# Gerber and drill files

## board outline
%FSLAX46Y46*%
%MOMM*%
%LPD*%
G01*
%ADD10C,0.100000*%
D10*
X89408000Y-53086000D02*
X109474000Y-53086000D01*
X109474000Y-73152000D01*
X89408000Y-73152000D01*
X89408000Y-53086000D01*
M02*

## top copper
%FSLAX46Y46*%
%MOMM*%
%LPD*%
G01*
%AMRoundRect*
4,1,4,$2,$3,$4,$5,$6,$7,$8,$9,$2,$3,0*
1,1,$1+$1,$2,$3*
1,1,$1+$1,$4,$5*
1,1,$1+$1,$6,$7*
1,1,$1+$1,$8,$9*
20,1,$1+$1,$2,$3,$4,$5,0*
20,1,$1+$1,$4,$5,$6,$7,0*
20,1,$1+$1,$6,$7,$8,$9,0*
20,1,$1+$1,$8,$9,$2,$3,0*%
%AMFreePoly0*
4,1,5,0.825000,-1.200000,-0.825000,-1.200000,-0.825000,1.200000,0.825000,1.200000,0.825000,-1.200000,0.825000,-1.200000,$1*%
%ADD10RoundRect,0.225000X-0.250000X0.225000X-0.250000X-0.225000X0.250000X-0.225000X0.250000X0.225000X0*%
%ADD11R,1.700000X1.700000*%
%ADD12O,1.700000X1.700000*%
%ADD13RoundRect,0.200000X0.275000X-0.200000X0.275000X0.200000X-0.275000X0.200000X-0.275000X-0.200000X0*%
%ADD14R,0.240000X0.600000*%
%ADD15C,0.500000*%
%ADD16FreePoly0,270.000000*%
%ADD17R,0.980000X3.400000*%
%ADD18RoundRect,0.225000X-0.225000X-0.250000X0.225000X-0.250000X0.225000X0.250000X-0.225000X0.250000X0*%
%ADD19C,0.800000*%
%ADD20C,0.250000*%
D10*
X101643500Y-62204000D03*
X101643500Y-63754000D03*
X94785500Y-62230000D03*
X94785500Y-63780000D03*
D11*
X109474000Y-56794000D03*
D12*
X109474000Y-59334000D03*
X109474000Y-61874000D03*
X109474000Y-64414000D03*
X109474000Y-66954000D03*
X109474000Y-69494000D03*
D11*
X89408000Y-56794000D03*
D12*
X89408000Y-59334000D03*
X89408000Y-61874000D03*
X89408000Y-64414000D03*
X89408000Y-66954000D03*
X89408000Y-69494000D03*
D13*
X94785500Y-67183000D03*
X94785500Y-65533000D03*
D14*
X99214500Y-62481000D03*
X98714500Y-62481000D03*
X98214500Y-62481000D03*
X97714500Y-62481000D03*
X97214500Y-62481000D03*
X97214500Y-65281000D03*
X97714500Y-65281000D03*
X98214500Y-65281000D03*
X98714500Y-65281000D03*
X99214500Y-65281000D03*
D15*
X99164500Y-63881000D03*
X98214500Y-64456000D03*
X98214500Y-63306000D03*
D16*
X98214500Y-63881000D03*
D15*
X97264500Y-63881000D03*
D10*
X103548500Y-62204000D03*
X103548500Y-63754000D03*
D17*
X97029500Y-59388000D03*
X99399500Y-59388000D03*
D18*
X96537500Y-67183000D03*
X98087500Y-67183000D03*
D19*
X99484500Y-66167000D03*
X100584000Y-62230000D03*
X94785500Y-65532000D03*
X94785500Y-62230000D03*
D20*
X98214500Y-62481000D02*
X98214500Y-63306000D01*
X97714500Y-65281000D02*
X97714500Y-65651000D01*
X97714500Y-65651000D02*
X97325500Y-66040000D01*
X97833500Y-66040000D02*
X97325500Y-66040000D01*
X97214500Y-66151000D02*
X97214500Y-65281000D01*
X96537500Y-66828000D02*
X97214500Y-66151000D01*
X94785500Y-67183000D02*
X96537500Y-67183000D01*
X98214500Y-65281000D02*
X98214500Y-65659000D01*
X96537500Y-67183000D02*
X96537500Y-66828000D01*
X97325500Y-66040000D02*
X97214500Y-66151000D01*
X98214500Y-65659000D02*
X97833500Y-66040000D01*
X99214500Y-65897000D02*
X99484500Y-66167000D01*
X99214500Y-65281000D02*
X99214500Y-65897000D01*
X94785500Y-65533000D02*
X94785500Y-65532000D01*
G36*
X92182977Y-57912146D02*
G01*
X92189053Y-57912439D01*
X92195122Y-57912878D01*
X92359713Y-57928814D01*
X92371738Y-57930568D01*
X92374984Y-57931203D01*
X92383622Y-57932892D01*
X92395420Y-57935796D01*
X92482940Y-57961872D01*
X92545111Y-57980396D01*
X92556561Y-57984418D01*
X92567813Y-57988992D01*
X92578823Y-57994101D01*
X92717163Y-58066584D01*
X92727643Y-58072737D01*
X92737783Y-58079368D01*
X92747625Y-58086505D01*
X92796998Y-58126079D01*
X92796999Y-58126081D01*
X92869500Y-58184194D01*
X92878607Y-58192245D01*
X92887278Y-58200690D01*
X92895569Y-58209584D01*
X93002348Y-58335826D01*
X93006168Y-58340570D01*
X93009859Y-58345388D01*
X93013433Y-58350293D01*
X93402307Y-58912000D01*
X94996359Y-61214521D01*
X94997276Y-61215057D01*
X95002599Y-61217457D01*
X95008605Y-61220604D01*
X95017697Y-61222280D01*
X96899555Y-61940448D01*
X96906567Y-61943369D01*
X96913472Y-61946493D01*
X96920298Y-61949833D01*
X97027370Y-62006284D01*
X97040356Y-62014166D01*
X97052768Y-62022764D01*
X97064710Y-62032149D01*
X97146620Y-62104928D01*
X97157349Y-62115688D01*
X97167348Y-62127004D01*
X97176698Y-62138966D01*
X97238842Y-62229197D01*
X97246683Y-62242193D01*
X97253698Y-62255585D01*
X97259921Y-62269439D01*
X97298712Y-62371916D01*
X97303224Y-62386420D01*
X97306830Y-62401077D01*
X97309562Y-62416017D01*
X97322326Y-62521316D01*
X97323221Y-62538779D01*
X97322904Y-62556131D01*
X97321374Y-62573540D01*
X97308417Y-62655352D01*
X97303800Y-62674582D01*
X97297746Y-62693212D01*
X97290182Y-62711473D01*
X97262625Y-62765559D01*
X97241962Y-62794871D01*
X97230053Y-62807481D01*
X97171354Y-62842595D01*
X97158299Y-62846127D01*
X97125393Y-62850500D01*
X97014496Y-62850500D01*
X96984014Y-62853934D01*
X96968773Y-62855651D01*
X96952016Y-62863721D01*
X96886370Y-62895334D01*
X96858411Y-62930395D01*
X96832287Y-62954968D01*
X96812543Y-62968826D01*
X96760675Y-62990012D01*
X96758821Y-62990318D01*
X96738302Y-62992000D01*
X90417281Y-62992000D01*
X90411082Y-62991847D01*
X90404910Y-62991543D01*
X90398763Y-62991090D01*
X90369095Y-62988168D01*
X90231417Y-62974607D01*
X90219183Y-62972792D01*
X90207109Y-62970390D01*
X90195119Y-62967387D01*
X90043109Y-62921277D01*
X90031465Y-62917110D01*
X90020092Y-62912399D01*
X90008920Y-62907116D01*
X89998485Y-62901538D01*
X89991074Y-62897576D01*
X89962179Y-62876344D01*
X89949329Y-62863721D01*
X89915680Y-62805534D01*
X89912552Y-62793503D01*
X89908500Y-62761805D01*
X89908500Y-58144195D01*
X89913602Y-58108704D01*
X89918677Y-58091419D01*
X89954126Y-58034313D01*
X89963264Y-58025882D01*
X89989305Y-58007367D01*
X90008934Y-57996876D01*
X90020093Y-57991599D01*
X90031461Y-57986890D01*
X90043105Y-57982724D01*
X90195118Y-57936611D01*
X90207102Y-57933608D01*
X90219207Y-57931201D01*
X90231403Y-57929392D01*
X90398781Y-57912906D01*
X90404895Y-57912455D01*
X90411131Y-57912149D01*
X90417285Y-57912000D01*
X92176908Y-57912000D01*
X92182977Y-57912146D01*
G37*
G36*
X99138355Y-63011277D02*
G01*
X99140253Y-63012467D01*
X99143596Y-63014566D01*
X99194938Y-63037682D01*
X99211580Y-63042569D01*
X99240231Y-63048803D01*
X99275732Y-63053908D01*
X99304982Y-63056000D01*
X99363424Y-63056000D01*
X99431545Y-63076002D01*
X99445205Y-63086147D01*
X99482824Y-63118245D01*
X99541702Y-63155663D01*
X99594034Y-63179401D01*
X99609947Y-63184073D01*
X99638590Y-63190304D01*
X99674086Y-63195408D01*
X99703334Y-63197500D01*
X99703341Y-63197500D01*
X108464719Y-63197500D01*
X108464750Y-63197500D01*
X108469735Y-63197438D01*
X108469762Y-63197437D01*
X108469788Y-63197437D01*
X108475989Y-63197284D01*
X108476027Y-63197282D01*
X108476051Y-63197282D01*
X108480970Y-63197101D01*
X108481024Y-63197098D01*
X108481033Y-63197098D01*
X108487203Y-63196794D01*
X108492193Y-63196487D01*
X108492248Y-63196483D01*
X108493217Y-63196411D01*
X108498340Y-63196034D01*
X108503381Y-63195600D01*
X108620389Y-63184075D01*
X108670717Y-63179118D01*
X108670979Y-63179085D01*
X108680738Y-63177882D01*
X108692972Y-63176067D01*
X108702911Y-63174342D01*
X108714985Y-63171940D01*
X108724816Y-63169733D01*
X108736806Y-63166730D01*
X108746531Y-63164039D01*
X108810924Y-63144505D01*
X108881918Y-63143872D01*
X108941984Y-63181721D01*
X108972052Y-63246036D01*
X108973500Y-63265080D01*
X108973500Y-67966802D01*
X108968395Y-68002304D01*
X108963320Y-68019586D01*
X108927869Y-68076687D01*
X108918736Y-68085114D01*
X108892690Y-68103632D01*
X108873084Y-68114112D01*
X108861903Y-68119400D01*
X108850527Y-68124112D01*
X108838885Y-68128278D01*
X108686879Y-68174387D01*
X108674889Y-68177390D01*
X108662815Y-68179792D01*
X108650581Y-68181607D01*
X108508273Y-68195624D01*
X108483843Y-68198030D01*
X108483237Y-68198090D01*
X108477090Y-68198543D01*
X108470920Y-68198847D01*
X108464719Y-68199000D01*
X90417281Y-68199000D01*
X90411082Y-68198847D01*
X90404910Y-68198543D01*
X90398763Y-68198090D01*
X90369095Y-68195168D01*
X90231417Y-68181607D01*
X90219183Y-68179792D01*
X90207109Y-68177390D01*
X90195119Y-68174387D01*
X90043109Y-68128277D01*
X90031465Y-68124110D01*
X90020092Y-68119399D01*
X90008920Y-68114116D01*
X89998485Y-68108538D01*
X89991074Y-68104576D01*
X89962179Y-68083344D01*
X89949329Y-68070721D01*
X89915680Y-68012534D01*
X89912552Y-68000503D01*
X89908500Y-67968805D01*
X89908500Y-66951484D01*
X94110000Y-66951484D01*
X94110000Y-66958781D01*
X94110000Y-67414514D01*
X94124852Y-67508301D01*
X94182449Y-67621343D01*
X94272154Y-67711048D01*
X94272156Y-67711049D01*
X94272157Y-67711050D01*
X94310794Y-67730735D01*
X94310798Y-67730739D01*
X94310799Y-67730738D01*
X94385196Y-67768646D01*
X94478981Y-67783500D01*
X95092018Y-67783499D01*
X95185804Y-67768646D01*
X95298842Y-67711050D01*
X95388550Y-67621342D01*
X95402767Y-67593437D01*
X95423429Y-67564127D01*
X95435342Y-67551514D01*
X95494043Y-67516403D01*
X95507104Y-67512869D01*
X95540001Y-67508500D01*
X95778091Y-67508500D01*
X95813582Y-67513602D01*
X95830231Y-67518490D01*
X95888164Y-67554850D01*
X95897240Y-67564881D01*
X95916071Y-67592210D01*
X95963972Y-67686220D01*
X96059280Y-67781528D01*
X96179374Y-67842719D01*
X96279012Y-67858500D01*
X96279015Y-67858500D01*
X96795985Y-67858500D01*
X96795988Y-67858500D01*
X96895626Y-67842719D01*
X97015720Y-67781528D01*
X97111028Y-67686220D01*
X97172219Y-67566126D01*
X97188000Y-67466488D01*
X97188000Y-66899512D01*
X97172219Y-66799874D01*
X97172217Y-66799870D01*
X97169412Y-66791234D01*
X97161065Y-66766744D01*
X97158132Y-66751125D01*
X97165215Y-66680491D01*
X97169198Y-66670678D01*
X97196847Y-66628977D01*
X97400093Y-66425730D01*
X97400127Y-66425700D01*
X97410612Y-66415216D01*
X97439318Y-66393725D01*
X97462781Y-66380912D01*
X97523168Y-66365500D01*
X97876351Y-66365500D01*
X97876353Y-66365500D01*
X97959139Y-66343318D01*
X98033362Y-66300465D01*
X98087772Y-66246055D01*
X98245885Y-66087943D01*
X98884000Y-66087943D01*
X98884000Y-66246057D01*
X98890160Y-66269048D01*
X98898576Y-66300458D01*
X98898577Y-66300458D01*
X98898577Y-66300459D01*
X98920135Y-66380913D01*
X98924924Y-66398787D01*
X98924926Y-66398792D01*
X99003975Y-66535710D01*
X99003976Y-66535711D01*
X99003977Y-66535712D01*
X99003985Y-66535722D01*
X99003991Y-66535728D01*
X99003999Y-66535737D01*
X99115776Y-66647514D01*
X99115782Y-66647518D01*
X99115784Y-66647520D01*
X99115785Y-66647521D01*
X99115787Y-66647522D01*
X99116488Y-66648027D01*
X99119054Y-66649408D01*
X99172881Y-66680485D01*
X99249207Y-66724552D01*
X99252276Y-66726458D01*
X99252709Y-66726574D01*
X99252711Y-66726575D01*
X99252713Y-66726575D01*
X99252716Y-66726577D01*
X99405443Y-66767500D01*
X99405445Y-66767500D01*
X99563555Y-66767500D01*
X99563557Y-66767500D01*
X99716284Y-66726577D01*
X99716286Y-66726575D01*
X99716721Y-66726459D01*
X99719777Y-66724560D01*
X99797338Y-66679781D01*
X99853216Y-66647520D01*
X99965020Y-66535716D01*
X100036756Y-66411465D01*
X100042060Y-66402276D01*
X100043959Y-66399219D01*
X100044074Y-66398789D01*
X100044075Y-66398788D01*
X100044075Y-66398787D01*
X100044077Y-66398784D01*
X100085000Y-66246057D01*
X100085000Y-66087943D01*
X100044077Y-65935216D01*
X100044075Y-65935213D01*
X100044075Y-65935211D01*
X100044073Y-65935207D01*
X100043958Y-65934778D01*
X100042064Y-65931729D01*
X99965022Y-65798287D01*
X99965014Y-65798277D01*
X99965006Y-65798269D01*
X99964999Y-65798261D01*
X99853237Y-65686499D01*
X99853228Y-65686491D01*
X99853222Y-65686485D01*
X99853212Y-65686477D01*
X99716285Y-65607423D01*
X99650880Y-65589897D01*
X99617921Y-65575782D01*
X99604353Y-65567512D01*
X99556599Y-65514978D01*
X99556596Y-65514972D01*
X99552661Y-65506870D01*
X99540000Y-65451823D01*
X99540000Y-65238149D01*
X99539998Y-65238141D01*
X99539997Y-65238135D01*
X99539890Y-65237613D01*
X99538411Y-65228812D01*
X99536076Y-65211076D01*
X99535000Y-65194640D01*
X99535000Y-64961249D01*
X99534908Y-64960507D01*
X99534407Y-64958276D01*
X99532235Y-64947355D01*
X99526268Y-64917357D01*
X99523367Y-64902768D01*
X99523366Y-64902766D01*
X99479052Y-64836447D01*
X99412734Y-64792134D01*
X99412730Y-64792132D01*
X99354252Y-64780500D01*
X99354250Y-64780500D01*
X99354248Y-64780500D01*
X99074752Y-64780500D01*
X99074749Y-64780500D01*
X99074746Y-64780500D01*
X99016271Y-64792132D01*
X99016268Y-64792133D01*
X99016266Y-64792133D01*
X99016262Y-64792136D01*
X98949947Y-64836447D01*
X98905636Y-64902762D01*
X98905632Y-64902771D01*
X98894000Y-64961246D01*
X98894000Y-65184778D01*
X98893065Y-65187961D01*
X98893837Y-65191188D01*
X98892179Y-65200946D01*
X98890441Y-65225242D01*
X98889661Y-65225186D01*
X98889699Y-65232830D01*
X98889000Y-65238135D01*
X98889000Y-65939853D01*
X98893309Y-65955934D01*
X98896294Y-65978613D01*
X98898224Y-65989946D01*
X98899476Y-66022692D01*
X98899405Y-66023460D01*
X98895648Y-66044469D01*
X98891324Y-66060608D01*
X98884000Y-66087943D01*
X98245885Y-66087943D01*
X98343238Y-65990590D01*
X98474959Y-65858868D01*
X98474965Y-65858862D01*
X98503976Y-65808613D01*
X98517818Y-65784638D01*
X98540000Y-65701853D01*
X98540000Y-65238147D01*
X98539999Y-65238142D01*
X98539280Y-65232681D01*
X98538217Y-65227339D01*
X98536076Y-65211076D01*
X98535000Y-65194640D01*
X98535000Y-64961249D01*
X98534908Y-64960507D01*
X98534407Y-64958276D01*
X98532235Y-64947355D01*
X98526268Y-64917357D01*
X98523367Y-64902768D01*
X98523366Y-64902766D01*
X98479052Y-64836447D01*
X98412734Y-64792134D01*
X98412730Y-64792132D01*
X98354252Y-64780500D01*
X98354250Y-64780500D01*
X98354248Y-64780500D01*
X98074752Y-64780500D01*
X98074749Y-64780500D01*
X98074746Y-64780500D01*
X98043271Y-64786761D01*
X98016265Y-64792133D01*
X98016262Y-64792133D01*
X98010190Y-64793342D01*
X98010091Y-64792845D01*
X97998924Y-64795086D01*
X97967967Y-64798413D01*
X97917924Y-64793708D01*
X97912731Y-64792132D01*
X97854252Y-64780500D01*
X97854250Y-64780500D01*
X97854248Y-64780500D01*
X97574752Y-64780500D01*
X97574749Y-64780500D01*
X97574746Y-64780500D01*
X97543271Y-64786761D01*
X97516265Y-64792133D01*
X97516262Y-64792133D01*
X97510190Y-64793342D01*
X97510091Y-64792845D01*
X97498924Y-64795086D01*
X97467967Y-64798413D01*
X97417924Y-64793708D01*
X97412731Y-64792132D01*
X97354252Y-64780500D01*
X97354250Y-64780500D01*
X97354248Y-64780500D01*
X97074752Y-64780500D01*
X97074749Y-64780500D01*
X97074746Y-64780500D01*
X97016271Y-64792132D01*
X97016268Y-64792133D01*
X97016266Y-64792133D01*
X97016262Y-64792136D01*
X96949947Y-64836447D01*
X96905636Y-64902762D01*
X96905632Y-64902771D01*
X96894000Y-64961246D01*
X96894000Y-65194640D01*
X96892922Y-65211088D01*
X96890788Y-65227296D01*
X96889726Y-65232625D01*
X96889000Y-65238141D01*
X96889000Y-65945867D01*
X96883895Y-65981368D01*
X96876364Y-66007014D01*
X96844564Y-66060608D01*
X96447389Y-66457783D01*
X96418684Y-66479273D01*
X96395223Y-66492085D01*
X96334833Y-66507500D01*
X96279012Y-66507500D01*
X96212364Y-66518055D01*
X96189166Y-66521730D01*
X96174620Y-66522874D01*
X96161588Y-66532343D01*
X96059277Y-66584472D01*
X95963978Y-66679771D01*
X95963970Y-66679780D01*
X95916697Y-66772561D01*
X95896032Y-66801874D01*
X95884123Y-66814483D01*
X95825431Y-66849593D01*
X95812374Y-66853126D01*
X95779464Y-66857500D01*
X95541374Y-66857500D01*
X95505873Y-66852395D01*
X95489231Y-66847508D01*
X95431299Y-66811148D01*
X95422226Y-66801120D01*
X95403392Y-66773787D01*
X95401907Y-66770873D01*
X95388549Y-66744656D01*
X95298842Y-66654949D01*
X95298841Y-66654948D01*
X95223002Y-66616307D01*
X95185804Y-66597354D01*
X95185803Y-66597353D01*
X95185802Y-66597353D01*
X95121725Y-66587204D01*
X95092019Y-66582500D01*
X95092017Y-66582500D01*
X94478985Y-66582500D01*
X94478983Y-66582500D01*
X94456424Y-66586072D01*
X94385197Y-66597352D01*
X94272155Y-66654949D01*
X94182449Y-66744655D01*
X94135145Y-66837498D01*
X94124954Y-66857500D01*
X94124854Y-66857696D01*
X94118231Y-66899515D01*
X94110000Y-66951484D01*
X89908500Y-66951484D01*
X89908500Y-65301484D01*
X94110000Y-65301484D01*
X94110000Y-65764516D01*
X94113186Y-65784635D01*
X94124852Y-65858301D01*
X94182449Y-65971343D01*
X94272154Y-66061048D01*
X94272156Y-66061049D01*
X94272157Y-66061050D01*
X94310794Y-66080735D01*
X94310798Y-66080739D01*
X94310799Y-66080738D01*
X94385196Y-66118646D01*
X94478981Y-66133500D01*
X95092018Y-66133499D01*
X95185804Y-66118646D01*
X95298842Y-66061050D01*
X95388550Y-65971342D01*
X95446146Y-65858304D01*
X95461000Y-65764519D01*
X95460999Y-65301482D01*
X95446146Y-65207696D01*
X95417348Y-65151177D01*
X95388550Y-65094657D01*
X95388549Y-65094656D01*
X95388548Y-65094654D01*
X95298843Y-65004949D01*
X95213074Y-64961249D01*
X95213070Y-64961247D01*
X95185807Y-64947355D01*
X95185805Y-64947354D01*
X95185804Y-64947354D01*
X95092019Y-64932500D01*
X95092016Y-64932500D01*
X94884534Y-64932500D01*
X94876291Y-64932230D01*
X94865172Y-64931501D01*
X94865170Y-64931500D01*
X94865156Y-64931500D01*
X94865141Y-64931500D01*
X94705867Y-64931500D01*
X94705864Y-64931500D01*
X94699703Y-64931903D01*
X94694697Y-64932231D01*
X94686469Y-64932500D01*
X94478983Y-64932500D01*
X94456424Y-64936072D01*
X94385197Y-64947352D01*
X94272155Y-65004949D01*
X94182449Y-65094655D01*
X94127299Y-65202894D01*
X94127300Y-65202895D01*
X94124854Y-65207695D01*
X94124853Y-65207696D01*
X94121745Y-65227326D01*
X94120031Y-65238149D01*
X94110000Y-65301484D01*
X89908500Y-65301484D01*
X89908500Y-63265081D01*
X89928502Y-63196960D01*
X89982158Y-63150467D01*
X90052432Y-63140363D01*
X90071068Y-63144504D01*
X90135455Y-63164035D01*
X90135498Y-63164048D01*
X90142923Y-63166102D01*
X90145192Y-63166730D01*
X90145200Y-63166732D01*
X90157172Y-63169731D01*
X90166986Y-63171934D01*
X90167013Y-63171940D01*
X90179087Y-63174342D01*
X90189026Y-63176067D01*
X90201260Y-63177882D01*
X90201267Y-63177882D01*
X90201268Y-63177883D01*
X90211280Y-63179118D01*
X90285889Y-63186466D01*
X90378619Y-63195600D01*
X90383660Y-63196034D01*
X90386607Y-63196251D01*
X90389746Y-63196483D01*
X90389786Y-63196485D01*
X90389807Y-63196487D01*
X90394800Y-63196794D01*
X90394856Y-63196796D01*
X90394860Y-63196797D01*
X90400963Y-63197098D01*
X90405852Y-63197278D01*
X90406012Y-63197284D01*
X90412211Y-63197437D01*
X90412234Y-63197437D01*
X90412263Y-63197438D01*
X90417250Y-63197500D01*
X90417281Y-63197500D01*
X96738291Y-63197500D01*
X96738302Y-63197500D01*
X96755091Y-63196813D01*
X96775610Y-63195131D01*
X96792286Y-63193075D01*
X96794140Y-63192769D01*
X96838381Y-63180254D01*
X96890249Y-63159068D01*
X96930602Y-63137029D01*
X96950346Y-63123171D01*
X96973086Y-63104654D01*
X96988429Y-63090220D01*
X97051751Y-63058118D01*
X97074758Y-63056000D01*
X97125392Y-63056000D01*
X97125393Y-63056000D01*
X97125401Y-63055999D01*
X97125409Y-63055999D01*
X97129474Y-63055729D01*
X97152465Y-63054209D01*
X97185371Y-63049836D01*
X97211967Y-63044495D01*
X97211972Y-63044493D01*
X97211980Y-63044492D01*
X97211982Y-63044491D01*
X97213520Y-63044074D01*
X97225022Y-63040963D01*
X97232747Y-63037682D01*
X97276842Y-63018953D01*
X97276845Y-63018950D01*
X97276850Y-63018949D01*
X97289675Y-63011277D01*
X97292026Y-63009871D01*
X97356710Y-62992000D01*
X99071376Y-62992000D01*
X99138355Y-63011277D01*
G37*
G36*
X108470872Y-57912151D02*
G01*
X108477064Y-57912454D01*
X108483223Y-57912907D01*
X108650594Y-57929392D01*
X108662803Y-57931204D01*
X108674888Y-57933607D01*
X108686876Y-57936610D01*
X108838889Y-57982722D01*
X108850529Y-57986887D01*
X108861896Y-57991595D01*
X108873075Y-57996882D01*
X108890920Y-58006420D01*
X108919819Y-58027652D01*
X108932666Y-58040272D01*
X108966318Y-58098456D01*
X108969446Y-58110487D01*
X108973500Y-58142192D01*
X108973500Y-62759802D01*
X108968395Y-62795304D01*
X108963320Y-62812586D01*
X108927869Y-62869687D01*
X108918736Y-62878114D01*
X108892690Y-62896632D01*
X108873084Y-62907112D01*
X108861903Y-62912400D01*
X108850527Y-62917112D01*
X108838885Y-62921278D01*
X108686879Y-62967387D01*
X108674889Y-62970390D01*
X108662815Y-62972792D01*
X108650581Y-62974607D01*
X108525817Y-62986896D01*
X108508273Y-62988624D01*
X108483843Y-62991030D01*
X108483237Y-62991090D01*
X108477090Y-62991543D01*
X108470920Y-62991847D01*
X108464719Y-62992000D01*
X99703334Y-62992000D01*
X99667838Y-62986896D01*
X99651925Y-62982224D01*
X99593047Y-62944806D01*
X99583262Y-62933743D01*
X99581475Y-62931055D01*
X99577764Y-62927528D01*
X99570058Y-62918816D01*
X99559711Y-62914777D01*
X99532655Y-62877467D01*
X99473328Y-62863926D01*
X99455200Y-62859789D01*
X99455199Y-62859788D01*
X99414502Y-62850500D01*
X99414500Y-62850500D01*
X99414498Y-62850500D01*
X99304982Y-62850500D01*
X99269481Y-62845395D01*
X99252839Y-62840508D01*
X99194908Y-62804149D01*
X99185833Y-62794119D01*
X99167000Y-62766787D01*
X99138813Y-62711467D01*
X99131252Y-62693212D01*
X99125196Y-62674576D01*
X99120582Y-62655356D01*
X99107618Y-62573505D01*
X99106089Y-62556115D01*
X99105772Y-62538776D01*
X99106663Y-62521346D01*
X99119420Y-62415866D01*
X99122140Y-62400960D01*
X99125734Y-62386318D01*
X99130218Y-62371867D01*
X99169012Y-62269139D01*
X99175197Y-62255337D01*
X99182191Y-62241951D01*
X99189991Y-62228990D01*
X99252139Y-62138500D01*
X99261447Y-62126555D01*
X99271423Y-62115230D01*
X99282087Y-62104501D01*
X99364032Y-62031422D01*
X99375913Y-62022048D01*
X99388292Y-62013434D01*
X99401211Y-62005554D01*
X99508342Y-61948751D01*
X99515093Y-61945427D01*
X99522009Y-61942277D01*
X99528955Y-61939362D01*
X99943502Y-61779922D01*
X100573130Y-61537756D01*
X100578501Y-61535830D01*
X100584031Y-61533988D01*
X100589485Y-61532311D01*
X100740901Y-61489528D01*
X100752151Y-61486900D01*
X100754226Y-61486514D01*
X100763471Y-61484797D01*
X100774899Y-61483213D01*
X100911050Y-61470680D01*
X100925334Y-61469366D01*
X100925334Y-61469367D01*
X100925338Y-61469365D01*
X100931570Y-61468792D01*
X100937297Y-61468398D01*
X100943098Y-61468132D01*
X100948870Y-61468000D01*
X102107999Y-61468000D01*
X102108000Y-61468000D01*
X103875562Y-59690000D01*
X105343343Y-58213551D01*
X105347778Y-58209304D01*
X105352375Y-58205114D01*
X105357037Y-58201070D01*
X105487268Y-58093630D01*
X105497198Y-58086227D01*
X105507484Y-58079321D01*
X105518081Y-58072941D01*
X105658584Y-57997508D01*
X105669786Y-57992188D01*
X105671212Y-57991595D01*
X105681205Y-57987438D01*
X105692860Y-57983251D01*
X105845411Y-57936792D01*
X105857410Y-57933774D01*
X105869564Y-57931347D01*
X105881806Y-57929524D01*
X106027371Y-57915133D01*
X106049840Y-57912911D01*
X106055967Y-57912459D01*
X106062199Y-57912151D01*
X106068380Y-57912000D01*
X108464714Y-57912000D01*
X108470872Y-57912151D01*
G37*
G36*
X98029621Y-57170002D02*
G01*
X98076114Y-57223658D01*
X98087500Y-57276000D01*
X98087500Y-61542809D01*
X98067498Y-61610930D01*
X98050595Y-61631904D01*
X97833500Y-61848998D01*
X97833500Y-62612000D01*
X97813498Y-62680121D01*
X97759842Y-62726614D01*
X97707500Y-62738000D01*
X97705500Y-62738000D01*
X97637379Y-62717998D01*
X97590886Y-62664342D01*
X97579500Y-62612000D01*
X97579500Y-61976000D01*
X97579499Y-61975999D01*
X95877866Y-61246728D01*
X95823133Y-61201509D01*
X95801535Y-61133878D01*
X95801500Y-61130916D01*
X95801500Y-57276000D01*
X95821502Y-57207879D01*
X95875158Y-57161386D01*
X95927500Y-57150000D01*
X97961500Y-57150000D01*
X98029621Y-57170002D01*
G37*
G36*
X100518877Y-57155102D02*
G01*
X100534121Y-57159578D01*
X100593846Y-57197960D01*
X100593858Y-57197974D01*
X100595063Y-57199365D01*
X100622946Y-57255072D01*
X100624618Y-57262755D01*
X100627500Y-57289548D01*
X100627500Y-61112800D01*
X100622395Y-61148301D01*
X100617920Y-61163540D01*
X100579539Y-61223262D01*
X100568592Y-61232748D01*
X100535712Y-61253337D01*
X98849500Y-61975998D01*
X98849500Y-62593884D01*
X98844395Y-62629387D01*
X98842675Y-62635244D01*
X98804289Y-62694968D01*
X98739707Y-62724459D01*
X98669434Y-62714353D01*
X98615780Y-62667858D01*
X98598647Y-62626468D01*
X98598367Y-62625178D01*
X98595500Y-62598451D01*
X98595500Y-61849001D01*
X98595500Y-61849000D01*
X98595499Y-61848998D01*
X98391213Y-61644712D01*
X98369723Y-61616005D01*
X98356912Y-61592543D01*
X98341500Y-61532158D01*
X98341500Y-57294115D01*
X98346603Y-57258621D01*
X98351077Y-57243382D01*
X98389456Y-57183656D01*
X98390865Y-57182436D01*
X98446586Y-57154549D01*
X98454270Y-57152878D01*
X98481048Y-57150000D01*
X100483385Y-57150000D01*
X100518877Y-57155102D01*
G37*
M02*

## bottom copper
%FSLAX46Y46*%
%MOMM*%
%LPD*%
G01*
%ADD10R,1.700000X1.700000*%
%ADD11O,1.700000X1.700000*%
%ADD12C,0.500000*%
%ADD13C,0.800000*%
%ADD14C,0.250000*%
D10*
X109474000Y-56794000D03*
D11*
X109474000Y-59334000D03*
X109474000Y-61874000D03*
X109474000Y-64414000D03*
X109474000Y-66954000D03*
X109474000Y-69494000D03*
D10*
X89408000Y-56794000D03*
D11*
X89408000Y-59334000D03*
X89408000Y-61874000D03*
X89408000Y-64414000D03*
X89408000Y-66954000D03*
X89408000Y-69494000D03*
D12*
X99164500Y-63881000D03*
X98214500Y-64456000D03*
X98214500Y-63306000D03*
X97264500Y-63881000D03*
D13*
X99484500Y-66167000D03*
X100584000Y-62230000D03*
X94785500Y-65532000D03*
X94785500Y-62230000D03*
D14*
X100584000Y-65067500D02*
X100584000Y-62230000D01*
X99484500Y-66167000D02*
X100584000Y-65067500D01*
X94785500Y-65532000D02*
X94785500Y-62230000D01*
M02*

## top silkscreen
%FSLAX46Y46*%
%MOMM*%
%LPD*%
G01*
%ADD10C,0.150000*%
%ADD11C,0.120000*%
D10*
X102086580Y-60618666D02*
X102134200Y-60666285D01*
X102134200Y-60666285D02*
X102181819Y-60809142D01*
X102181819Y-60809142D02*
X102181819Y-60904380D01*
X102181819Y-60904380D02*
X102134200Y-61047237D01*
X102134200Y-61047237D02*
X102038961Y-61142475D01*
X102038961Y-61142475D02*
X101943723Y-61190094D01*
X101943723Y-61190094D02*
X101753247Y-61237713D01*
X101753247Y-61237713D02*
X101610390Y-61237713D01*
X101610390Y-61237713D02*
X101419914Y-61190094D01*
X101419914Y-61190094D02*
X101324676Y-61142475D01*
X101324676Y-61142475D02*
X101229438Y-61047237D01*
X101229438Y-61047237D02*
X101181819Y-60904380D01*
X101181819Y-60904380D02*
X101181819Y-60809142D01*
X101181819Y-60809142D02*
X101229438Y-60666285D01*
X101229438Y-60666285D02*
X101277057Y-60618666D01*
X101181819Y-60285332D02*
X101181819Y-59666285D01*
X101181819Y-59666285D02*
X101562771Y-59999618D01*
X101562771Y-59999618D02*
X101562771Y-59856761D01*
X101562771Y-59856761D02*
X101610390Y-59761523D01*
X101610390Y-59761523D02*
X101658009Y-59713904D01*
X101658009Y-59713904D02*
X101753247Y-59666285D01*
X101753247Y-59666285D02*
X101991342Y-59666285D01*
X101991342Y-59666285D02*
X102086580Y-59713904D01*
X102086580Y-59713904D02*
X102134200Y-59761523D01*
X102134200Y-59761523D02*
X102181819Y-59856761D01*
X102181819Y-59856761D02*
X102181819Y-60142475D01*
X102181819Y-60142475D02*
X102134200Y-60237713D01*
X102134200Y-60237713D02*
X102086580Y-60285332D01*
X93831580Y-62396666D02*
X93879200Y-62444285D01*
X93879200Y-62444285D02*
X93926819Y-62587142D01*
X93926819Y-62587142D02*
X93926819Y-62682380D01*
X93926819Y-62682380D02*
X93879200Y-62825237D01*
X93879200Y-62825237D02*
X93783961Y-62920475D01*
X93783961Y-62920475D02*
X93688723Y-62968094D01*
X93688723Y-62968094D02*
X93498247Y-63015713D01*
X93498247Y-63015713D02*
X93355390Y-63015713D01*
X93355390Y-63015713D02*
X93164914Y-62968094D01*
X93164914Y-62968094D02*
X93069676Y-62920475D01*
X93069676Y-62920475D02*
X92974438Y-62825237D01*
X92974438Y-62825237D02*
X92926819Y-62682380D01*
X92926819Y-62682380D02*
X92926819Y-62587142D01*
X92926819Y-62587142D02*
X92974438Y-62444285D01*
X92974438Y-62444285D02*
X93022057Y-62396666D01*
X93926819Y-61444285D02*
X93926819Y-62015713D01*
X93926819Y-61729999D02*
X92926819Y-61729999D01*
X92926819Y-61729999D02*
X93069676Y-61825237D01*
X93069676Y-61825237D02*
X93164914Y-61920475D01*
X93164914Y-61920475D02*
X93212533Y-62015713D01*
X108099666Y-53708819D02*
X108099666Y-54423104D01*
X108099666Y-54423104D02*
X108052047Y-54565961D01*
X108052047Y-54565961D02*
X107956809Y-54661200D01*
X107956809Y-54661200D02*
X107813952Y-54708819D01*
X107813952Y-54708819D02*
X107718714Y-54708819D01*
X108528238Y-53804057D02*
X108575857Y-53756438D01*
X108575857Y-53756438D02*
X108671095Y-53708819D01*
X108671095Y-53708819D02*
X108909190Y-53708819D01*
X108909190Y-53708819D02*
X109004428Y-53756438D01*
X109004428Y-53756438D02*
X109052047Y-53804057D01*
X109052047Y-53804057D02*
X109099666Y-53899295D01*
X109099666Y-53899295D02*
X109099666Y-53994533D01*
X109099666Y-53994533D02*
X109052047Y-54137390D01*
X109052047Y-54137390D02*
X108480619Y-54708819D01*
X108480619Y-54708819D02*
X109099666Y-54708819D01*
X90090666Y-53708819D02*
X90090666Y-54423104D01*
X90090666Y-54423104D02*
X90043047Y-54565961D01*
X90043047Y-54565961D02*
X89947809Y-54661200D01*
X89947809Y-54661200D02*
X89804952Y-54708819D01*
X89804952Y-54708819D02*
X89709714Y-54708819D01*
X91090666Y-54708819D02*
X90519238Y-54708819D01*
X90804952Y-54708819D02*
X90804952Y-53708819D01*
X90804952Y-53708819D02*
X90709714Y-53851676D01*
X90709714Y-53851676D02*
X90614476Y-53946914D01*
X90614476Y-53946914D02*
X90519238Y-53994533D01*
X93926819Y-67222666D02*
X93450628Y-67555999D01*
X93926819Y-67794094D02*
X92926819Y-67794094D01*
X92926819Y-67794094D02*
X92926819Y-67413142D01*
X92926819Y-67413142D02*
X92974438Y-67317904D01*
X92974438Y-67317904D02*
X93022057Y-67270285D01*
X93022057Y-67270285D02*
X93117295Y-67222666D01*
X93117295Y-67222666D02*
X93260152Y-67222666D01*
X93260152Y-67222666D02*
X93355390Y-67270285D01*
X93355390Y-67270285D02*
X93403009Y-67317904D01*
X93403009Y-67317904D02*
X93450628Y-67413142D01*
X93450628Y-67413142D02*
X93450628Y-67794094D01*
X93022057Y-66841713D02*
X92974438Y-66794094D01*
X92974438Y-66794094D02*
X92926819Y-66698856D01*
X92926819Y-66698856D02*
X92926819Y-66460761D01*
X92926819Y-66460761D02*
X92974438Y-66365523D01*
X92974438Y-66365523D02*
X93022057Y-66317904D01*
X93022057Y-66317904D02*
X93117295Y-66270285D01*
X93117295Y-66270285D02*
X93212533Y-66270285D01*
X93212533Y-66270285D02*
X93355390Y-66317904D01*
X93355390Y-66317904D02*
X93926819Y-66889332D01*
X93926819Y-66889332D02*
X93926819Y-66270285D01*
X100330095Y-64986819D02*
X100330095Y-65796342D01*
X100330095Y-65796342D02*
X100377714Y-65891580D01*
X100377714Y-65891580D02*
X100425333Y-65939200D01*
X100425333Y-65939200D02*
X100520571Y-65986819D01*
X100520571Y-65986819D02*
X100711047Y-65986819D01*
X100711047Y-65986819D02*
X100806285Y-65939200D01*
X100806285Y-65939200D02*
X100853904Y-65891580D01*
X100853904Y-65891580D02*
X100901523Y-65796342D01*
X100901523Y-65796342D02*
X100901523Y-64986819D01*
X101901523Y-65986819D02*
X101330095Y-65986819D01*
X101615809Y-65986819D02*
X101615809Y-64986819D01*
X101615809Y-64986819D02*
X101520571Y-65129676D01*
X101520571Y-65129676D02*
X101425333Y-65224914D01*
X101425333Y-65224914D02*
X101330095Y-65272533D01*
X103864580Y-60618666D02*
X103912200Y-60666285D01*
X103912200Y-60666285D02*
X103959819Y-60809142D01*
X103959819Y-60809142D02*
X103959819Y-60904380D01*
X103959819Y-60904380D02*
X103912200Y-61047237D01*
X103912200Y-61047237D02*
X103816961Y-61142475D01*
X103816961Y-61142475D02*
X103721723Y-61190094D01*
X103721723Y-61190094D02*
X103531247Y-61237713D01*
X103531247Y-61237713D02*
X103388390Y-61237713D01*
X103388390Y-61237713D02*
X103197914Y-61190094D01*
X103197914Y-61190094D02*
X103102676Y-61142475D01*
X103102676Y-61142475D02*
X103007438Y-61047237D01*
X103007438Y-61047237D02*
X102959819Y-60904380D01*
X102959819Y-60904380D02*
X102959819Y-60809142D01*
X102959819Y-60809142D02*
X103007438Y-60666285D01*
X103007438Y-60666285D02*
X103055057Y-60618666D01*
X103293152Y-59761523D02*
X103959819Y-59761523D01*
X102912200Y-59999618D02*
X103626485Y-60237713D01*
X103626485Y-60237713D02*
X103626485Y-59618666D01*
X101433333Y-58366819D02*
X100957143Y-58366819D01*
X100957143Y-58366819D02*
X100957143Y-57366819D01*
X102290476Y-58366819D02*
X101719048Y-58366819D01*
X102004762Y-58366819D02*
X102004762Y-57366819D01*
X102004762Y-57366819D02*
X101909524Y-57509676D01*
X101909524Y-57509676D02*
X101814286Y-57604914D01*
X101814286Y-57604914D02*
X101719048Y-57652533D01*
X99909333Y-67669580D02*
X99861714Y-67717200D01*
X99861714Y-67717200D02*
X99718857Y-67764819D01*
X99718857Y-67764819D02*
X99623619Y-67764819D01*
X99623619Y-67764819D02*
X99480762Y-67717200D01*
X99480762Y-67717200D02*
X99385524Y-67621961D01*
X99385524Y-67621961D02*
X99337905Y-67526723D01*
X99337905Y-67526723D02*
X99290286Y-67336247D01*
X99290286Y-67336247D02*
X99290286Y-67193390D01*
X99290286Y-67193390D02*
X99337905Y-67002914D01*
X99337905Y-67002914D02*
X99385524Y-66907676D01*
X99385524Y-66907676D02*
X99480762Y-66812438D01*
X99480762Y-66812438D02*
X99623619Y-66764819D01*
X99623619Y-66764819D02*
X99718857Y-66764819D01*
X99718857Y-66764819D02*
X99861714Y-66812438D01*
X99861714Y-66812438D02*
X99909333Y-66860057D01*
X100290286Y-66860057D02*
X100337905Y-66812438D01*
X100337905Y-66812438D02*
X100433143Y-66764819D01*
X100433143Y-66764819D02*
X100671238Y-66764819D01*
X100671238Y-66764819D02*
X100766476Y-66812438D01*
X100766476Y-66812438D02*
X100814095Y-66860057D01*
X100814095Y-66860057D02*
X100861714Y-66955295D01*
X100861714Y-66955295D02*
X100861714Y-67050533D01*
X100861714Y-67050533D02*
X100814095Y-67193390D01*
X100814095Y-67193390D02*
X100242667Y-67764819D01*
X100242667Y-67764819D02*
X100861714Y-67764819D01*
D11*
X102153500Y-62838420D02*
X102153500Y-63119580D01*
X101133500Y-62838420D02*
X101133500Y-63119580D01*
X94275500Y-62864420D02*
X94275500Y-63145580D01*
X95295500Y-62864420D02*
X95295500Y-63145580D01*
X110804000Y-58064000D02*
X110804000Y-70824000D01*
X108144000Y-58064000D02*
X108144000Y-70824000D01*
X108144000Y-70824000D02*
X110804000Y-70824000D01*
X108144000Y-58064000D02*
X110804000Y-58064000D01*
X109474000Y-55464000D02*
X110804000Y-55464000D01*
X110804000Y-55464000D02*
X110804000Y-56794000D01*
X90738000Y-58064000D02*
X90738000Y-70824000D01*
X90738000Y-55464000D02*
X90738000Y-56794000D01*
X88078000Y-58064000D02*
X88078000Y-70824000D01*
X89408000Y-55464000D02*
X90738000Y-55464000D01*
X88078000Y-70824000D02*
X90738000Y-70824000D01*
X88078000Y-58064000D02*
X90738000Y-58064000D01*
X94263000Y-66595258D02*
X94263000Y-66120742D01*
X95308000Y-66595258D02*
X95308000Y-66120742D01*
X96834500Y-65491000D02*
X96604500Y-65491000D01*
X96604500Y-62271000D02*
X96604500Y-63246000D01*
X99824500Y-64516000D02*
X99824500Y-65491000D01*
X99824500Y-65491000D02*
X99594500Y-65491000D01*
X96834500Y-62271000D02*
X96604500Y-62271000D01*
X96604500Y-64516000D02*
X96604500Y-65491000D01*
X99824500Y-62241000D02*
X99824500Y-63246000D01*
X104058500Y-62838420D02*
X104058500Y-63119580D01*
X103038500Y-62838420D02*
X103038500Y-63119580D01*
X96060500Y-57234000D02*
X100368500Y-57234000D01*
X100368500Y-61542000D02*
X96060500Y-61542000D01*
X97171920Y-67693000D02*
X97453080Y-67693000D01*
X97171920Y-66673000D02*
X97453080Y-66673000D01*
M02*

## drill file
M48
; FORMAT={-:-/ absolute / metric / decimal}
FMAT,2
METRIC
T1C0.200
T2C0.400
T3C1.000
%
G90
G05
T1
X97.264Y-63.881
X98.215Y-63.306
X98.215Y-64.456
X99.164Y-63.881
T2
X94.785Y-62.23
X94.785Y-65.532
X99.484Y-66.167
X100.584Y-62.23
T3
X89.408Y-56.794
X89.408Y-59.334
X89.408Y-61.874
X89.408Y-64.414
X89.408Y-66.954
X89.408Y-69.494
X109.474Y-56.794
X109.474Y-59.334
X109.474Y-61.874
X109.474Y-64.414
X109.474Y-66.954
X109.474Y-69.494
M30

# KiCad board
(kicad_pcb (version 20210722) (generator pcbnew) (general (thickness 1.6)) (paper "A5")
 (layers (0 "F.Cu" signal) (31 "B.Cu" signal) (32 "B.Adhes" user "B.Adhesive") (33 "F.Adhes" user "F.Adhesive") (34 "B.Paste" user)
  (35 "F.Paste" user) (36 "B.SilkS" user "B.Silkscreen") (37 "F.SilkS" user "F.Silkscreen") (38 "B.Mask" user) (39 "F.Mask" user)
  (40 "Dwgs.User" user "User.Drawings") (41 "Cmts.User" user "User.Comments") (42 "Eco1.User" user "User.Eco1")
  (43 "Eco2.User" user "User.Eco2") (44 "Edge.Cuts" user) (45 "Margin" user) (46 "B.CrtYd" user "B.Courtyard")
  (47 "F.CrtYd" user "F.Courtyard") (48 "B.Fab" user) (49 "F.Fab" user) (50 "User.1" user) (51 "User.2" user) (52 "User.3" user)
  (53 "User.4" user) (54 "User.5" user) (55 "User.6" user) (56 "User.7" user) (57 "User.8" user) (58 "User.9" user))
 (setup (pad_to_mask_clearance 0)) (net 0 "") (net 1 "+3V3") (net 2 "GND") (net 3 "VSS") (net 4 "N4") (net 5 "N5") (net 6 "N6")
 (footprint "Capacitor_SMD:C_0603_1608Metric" (layer "F.Cu") (at 101.6435 62.979 -90)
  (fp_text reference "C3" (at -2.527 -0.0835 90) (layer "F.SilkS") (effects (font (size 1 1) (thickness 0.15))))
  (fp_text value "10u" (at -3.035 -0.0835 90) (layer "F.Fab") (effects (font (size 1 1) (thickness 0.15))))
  (fp_line (start -0.14058 -0.51) (end 0.14058 -0.51) (layer "F.SilkS") (width 0.12))
  (fp_line (start -0.14058 0.51) (end 0.14058 0.51) (layer "F.SilkS") (width 0.12))
  (pad "1" smd roundrect locked (at -0.775 0 270) (size 0.9 0.95) (layers "F.Cu" "F.Paste" "F.Mask") (roundrect_rratio 0.25) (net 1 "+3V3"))
  (pad "2" smd roundrect locked (at 0.775 0 270) (size 0.9 0.95) (layers "F.Cu" "F.Paste" "F.Mask") (roundrect_rratio 0.25) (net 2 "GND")))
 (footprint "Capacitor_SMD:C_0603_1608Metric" (layer "F.Cu") (at 94.7855 63.005 -90)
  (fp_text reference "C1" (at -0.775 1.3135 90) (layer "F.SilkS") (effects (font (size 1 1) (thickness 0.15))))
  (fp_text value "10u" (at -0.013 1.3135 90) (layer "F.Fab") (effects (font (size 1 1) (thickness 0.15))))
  (fp_line (start -0.14058 0.51) (end 0.14058 0.51) (layer "F.SilkS") (width 0.12))
  (fp_line (start -0.14058 -0.51) (end 0.14058 -0.51) (layer "F.SilkS") (width 0.12))
  (pad "1" smd roundrect locked (at -0.775 0 270) (size 0.9 0.95) (layers "F.Cu" "F.Paste" "F.Mask") (roundrect_rratio 0.25) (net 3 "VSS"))
  (pad "2" smd roundrect locked (at 0.775 0 270) (size 0.9 0.95) (layers "F.Cu" "F.Paste" "F.Mask") (roundrect_rratio 0.25) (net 2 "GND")))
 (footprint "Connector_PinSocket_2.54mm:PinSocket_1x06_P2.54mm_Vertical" (layer "F.Cu") (at 109.474 56.794)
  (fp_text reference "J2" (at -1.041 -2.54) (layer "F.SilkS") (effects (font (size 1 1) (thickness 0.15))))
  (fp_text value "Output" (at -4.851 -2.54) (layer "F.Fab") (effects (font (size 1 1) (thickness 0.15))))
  (fp_line (start 1.33 1.27) (end 1.33 14.03) (layer "F.SilkS") (width 0.12))
  (fp_line (start -1.33 1.27) (end -1.33 14.03) (layer "F.SilkS") (width 0.12))
  (fp_line (start -1.33 14.03) (end 1.33 14.03) (layer "F.SilkS") (width 0.12))
  (fp_line (start -1.33 1.27) (end 1.33 1.27) (layer "F.SilkS") (width 0.12))
  (fp_line (start 0 -1.33) (end 1.33 -1.33) (layer "F.SilkS") (width 0.12))
  (fp_line (start 1.33 -1.33) (end 1.33 0) (layer "F.SilkS") (width 0.12))
  (pad "1" thru_hole rect locked (at 0 0) (size 1.7 1.7) (drill 1) (layers *.Cu *.Mask))
  (pad "2" thru_hole oval locked (at 0 2.54) (size 1.7 1.7) (drill 1) (layers *.Cu *.Mask) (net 1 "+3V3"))
  (pad "3" thru_hole oval locked (at 0 5.08) (size 1.7 1.7) (drill 1) (layers *.Cu *.Mask) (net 1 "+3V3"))
  (pad "4" thru_hole oval locked (at 0 7.62) (size 1.7 1.7) (drill 1) (layers *.Cu *.Mask) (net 2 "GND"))
  (pad "5" thru_hole oval locked (at 0 10.16) (size 1.7 1.7) (drill 1) (layers *.Cu *.Mask) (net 2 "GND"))
  (pad "6" thru_hole oval locked (at 0 12.7) (size 1.7 1.7) (drill 1) (layers *.Cu *.Mask)))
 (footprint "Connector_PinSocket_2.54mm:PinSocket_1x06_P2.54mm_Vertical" (layer "F.Cu") (at 89.408 56.794)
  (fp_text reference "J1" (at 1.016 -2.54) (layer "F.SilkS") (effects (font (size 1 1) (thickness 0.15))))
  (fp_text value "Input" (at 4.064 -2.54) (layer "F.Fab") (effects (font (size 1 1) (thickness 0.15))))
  (fp_line (start 1.33 1.27) (end 1.33 14.03) (layer "F.SilkS") (width 0.12))
  (fp_line (start 1.33 -1.33) (end 1.33 0) (layer "F.SilkS") (width 0.12))
  (fp_line (start -1.33 1.27) (end -1.33 14.03) (layer "F.SilkS") (width 0.12))
  (fp_line (start 0 -1.33) (end 1.33 -1.33) (layer "F.SilkS") (width 0.12))
  (fp_line (start -1.33 14.03) (end 1.33 14.03) (layer "F.SilkS") (width 0.12))
  (fp_line (start -1.33 1.27) (end 1.33 1.27) (layer "F.SilkS") (width 0.12))
  (pad "1" thru_hole rect locked (at 0 0) (size 1.7 1.7) (drill 1) (layers *.Cu *.Mask))
  (pad "2" thru_hole oval locked (at 0 2.54) (size 1.7 1.7) (drill 1) (layers *.Cu *.Mask) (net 3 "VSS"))
  (pad "3" thru_hole oval locked (at 0 5.08) (size 1.7 1.7) (drill 1) (layers *.Cu *.Mask) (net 3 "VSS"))
  (pad "4" thru_hole oval locked (at 0 7.62) (size 1.7 1.7) (drill 1) (layers *.Cu *.Mask) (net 2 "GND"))
  (pad "5" thru_hole oval locked (at 0 10.16) (size 1.7 1.7) (drill 1) (layers *.Cu *.Mask) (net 2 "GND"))
  (pad "6" thru_hole oval locked (at 0 12.7) (size 1.7 1.7) (drill 1) (layers *.Cu *.Mask)))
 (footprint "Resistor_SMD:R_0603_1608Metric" (layer "F.Cu") (at 94.7855 66.358 90)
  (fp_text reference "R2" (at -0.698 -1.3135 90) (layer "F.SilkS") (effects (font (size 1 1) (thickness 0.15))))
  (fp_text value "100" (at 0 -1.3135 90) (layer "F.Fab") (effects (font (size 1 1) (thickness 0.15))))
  (fp_line (start -0.237258 -0.5225) (end 0.237258 -0.5225) (layer "F.SilkS") (width 0.12))
  (fp_line (start -0.237258 0.5225) (end 0.237258 0.5225) (layer "F.SilkS") (width 0.12))
  (pad "1" smd roundrect locked (at -0.825 0 90) (size 0.8 0.95) (layers "F.Cu" "F.Paste" "F.Mask") (roundrect_rratio 0.25) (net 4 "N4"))
  (pad "2" smd roundrect locked (at 0.825 0 90) (size 0.8 0.95) (layers "F.Cu" "F.Paste" "F.Mask") (roundrect_rratio 0.25) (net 3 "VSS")))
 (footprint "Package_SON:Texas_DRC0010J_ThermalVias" (layer "F.Cu") (at 98.2145 63.881 -90)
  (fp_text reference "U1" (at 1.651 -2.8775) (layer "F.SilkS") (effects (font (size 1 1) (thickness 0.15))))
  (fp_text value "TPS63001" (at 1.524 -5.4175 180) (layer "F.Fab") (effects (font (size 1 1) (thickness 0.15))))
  (fp_line (start 1.61 1.38) (end 1.61 1.61) (layer "F.SilkS") (width 0.12))
  (fp_line (start -1.61 1.61) (end -0.635 1.61) (layer "F.SilkS") (width 0.12))
  (fp_line (start 0.635 -1.61) (end 1.61 -1.61) (layer "F.SilkS") (width 0.12))
  (fp_line (start 1.61 -1.61) (end 1.61 -1.38) (layer "F.SilkS") (width 0.12))
  (fp_line (start -1.61 1.38) (end -1.61 1.61) (layer "F.SilkS") (width 0.12))
  (fp_line (start 0.635 1.61) (end 1.61 1.61) (layer "F.SilkS") (width 0.12))
  (fp_line (start -1.64 -1.61) (end -0.635 -1.61) (layer "F.SilkS") (width 0.12))
  (pad "" smd roundrect locked (at 0 -0.63 270) (size 1.5 1.06) (layers "F.Paste") (roundrect_rratio 0.1) (zone_connect 0))
  (pad "" smd roundrect locked (at 0.25 1.53 270) (size 0.25 0.34) (layers "F.Paste") (roundrect_rratio 0.1) (zone_connect 0))
  (pad "" smd roundrect locked (at -0.25 -1.53 270) (size 0.25 0.34) (layers "F.Paste") (roundrect_rratio 0.1) (zone_connect 0))
  (pad "" smd roundrect locked (at 0 0.63 270) (size 1.5 1.06) (layers "F.Paste") (roundrect_rratio 0.1) (zone_connect 0))
  (pad "" smd roundrect locked (at -0.25 1.53 270) (size 0.25 0.34) (layers "F.Paste") (roundrect_rratio 0.1) (zone_connect 0))
  (pad "" smd roundrect locked (at 0.25 -1.53 270) (size 0.25 0.34) (layers "F.Paste") (roundrect_rratio 0.1) (zone_connect 0))
  (pad "1" smd rect locked (at -1.4 -1 270) (size 0.6 0.24) (layers "F.Cu" "F.Paste" "F.Mask") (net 1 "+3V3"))
  (pad "2" smd rect locked (at -1.4 -0.5 270) (size 0.6 0.24) (layers "F.Cu" "F.Paste" "F.Mask") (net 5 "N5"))
  (pad "3" smd rect locked (at -1.4 0 270) (size 0.6 0.24) (layers "F.Cu" "F.Paste" "F.Mask") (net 2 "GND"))
  (pad "4" smd rect locked (at -1.4 0.5 270) (size 0.6 0.24) (layers "F.Cu" "F.Paste" "F.Mask") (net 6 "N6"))
  (pad "5" smd rect locked (at -1.4 1 270) (size 0.6 0.24) (layers "F.Cu" "F.Paste" "F.Mask") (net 3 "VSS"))
  (pad "6" smd rect locked (at 1.4 1 270) (size 0.6 0.24) (layers "F.Cu" "F.Paste" "F.Mask") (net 4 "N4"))
  (pad "7" smd rect locked (at 1.4 0.5 270) (size 0.6 0.24) (layers "F.Cu" "F.Paste" "F.Mask") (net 4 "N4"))
  (pad "8" smd rect locked (at 1.4 0 270) (size 0.6 0.24) (layers "F.Cu" "F.Paste" "F.Mask") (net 4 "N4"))
  (pad "9" smd rect locked (at 1.4 -0.5 270) (size 0.6 0.24) (layers "F.Cu" "F.Paste" "F.Mask") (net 2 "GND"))
  (pad "10" smd rect locked (at 1.4 -1 270) (size 0.6 0.24) (layers "F.Cu" "F.Paste" "F.Mask") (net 1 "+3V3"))
  (pad "11" thru_hole circle locked (at 0 -0.95 270) (size 0.5 0.5) (drill 0.2) (layers *.Cu) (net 2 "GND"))
  (pad "11" thru_hole circle locked (at 0.575 0 270) (size 0.5 0.5) (drill 0.2) (layers *.Cu) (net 2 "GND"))
  (pad "11" thru_hole circle locked (at -0.575 0 270) (size 0.5 0.5) (drill 0.2) (layers *.Cu) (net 2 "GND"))
  (pad "11" smd custom locked (at 0 0 270) (size 1.65 2.4) (layers "F.Cu" "F.Mask") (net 2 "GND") (zone_connect 2)
   (options (clearance outline) (anchor rect)) (primitives))
  (pad "11" thru_hole circle locked (at 0 0.95 270) (size 0.5 0.5) (drill 0.2) (layers *.Cu) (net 2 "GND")))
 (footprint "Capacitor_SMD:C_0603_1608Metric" (layer "F.Cu") (at 103.5485 62.979 -90)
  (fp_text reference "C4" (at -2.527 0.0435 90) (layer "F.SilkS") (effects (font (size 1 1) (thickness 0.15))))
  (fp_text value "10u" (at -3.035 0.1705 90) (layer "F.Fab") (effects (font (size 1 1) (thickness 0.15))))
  (fp_line (start -0.14058 -0.51) (end 0.14058 -0.51) (layer "F.SilkS") (width 0.12))
  (fp_line (start -0.14058 0.51) (end 0.14058 0.51) (layer "F.SilkS") (width 0.12))
  (pad "1" smd roundrect locked (at -0.775 0 270) (size 0.9 0.95) (layers "F.Cu" "F.Paste" "F.Mask") (roundrect_rratio 0.25) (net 1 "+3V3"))
  (pad "2" smd roundrect locked (at 0.775 0 270) (size 0.9 0.95) (layers "F.Cu" "F.Paste" "F.Mask") (roundrect_rratio 0.25) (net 2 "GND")))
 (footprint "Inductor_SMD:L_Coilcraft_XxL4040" (layer "F.Cu") (at 98.2145 59.388)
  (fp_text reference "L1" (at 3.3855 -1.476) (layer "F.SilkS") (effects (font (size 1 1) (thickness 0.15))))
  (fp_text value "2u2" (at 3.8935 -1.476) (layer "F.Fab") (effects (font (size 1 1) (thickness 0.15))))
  (fp_line (start -2.154 -2.154) (end 2.154 -2.154) (layer "F.SilkS") (width 0.12))
  (fp_line (start 2.154 2.154) (end -2.154 2.154) (layer "F.SilkS") (width 0.12))
  (pad "1" smd rect locked (at -1.185 0) (size 0.98 3.4) (layers "F.Cu" "F.Paste" "F.Mask") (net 6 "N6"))
  (pad "2" smd rect locked (at 1.185 0) (size 0.98 3.4) (layers "F.Cu" "F.Paste" "F.Mask") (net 5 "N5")))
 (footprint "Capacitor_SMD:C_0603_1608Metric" (layer "F.Cu") (at 97.3125 67.183)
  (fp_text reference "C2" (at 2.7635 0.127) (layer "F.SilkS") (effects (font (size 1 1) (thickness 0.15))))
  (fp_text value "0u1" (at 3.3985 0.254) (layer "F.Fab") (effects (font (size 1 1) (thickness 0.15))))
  (fp_line (start -0.14058 0.51) (end 0.14058 0.51) (layer "F.SilkS") (width 0.12))
  (fp_line (start -0.14058 -0.51) (end 0.14058 -0.51) (layer "F.SilkS") (width 0.12))
  (pad "1" smd roundrect locked (at -0.775 0) (size 0.9 0.95) (layers "F.Cu" "F.Paste" "F.Mask") (roundrect_rratio 0.25) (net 4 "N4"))
  (pad "2" smd roundrect locked (at 0.775 0) (size 0.9 0.95) (layers "F.Cu" "F.Paste" "F.Mask") (roundrect_rratio 0.25) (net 2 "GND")))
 (gr_rect (start 109.474 73.152) (end 89.408 53.086) (layer "Edge.Cuts") (width 0.1) (fill none))
 (segment (start 98.2145 62.481) (end 98.2145 63.306) (width 0.25) (layer "F.Cu") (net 2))
 (segment (start 97.7145 65.281) (end 97.7145 65.651) (width 0.25) (layer "F.Cu") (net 4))
 (segment (start 97.7145 65.651) (end 97.3255 66.04) (width 0.25) (layer "F.Cu") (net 4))
 (segment (start 97.8335 66.04) (end 97.3255 66.04) (width 0.25) (layer "F.Cu") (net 4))
 (segment (start 97.2145 66.151) (end 97.2145 65.281) (width 0.25) (layer "F.Cu") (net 4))
 (segment (start 96.5375 66.828) (end 97.2145 66.151) (width 0.25) (layer "F.Cu") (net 4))
 (segment (start 94.7855 67.183) (end 96.5375 67.183) (width 0.25) (layer "F.Cu") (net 4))
 (segment (start 98.2145 65.281) (end 98.2145 65.659) (width 0.25) (layer "F.Cu") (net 4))
 (segment (start 96.5375 67.183) (end 96.5375 66.828) (width 0.25) (layer "F.Cu") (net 4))
 (segment (start 97.3255 66.04) (end 97.2145 66.151) (width 0.25) (layer "F.Cu") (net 4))
 (segment (start 98.2145 65.659) (end 97.8335 66.04) (width 0.25) (layer "F.Cu") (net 4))
 (segment (start 99.2145 65.897) (end 99.4845 66.167) (width 0.25) (layer "F.Cu") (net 1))
 (segment (start 99.2145 65.281) (end 99.2145 65.897) (width 0.25) (layer "F.Cu") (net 1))
 (via (at 99.4845 66.167) (size 0.8) (drill 0.4) (layers "F.Cu" "B.Cu") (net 1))
 (via (at 100.584 62.23) (size 0.8) (drill 0.4) (layers "F.Cu" "B.Cu") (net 1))
 (segment (start 100.584 65.0675) (end 100.584 62.23) (width 0.25) (layer "B.Cu") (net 1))
 (segment (start 99.4845 66.167) (end 100.584 65.0675) (width 0.25) (layer "B.Cu") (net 1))
 (segment (start 94.7855 65.533) (end 94.7855 65.532) (width 0.25) (layer "F.Cu") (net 3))
 (via (at 94.7855 65.532) (size 0.8) (drill 0.4) (layers "F.Cu" "B.Cu") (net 3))
 (via (at 94.7855 62.23) (size 0.8) (drill 0.4) (layers "F.Cu" "B.Cu") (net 3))
 (segment (start 94.7855 65.532) (end 94.7855 62.23) (width 0.25) (layer "B.Cu") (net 3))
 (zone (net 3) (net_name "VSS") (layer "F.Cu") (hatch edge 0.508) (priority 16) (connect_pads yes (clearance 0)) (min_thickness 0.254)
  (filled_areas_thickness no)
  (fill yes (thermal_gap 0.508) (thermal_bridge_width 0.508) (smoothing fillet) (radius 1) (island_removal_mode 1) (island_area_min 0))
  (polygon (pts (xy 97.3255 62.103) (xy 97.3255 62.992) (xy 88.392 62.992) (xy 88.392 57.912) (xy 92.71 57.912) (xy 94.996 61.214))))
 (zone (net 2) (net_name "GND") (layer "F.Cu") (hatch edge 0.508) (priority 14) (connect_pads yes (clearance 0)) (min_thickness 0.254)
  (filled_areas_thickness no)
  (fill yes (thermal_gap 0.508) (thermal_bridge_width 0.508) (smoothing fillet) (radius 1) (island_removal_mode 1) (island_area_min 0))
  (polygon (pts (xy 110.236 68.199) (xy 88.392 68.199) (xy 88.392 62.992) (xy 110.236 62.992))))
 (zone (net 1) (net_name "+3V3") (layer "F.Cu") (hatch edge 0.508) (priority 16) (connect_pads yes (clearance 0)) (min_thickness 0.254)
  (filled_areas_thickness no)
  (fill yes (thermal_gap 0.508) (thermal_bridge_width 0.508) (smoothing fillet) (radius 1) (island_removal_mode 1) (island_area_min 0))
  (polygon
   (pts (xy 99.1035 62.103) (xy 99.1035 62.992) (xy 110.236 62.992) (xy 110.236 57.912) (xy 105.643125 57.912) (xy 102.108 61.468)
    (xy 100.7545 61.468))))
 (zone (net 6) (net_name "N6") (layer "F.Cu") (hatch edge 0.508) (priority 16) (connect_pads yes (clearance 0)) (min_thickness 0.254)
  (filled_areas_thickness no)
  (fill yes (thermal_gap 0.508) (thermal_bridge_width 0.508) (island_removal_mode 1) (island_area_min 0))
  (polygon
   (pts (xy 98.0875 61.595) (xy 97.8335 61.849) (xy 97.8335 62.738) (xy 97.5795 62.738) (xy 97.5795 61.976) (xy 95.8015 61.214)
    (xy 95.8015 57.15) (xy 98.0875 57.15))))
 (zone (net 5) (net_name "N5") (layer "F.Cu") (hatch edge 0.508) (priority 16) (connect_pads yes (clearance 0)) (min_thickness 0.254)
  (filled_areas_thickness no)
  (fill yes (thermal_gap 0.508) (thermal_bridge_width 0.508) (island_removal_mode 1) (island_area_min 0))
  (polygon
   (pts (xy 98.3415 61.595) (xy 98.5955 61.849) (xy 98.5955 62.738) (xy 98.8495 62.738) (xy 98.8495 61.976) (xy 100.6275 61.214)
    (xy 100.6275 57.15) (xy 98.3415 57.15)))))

